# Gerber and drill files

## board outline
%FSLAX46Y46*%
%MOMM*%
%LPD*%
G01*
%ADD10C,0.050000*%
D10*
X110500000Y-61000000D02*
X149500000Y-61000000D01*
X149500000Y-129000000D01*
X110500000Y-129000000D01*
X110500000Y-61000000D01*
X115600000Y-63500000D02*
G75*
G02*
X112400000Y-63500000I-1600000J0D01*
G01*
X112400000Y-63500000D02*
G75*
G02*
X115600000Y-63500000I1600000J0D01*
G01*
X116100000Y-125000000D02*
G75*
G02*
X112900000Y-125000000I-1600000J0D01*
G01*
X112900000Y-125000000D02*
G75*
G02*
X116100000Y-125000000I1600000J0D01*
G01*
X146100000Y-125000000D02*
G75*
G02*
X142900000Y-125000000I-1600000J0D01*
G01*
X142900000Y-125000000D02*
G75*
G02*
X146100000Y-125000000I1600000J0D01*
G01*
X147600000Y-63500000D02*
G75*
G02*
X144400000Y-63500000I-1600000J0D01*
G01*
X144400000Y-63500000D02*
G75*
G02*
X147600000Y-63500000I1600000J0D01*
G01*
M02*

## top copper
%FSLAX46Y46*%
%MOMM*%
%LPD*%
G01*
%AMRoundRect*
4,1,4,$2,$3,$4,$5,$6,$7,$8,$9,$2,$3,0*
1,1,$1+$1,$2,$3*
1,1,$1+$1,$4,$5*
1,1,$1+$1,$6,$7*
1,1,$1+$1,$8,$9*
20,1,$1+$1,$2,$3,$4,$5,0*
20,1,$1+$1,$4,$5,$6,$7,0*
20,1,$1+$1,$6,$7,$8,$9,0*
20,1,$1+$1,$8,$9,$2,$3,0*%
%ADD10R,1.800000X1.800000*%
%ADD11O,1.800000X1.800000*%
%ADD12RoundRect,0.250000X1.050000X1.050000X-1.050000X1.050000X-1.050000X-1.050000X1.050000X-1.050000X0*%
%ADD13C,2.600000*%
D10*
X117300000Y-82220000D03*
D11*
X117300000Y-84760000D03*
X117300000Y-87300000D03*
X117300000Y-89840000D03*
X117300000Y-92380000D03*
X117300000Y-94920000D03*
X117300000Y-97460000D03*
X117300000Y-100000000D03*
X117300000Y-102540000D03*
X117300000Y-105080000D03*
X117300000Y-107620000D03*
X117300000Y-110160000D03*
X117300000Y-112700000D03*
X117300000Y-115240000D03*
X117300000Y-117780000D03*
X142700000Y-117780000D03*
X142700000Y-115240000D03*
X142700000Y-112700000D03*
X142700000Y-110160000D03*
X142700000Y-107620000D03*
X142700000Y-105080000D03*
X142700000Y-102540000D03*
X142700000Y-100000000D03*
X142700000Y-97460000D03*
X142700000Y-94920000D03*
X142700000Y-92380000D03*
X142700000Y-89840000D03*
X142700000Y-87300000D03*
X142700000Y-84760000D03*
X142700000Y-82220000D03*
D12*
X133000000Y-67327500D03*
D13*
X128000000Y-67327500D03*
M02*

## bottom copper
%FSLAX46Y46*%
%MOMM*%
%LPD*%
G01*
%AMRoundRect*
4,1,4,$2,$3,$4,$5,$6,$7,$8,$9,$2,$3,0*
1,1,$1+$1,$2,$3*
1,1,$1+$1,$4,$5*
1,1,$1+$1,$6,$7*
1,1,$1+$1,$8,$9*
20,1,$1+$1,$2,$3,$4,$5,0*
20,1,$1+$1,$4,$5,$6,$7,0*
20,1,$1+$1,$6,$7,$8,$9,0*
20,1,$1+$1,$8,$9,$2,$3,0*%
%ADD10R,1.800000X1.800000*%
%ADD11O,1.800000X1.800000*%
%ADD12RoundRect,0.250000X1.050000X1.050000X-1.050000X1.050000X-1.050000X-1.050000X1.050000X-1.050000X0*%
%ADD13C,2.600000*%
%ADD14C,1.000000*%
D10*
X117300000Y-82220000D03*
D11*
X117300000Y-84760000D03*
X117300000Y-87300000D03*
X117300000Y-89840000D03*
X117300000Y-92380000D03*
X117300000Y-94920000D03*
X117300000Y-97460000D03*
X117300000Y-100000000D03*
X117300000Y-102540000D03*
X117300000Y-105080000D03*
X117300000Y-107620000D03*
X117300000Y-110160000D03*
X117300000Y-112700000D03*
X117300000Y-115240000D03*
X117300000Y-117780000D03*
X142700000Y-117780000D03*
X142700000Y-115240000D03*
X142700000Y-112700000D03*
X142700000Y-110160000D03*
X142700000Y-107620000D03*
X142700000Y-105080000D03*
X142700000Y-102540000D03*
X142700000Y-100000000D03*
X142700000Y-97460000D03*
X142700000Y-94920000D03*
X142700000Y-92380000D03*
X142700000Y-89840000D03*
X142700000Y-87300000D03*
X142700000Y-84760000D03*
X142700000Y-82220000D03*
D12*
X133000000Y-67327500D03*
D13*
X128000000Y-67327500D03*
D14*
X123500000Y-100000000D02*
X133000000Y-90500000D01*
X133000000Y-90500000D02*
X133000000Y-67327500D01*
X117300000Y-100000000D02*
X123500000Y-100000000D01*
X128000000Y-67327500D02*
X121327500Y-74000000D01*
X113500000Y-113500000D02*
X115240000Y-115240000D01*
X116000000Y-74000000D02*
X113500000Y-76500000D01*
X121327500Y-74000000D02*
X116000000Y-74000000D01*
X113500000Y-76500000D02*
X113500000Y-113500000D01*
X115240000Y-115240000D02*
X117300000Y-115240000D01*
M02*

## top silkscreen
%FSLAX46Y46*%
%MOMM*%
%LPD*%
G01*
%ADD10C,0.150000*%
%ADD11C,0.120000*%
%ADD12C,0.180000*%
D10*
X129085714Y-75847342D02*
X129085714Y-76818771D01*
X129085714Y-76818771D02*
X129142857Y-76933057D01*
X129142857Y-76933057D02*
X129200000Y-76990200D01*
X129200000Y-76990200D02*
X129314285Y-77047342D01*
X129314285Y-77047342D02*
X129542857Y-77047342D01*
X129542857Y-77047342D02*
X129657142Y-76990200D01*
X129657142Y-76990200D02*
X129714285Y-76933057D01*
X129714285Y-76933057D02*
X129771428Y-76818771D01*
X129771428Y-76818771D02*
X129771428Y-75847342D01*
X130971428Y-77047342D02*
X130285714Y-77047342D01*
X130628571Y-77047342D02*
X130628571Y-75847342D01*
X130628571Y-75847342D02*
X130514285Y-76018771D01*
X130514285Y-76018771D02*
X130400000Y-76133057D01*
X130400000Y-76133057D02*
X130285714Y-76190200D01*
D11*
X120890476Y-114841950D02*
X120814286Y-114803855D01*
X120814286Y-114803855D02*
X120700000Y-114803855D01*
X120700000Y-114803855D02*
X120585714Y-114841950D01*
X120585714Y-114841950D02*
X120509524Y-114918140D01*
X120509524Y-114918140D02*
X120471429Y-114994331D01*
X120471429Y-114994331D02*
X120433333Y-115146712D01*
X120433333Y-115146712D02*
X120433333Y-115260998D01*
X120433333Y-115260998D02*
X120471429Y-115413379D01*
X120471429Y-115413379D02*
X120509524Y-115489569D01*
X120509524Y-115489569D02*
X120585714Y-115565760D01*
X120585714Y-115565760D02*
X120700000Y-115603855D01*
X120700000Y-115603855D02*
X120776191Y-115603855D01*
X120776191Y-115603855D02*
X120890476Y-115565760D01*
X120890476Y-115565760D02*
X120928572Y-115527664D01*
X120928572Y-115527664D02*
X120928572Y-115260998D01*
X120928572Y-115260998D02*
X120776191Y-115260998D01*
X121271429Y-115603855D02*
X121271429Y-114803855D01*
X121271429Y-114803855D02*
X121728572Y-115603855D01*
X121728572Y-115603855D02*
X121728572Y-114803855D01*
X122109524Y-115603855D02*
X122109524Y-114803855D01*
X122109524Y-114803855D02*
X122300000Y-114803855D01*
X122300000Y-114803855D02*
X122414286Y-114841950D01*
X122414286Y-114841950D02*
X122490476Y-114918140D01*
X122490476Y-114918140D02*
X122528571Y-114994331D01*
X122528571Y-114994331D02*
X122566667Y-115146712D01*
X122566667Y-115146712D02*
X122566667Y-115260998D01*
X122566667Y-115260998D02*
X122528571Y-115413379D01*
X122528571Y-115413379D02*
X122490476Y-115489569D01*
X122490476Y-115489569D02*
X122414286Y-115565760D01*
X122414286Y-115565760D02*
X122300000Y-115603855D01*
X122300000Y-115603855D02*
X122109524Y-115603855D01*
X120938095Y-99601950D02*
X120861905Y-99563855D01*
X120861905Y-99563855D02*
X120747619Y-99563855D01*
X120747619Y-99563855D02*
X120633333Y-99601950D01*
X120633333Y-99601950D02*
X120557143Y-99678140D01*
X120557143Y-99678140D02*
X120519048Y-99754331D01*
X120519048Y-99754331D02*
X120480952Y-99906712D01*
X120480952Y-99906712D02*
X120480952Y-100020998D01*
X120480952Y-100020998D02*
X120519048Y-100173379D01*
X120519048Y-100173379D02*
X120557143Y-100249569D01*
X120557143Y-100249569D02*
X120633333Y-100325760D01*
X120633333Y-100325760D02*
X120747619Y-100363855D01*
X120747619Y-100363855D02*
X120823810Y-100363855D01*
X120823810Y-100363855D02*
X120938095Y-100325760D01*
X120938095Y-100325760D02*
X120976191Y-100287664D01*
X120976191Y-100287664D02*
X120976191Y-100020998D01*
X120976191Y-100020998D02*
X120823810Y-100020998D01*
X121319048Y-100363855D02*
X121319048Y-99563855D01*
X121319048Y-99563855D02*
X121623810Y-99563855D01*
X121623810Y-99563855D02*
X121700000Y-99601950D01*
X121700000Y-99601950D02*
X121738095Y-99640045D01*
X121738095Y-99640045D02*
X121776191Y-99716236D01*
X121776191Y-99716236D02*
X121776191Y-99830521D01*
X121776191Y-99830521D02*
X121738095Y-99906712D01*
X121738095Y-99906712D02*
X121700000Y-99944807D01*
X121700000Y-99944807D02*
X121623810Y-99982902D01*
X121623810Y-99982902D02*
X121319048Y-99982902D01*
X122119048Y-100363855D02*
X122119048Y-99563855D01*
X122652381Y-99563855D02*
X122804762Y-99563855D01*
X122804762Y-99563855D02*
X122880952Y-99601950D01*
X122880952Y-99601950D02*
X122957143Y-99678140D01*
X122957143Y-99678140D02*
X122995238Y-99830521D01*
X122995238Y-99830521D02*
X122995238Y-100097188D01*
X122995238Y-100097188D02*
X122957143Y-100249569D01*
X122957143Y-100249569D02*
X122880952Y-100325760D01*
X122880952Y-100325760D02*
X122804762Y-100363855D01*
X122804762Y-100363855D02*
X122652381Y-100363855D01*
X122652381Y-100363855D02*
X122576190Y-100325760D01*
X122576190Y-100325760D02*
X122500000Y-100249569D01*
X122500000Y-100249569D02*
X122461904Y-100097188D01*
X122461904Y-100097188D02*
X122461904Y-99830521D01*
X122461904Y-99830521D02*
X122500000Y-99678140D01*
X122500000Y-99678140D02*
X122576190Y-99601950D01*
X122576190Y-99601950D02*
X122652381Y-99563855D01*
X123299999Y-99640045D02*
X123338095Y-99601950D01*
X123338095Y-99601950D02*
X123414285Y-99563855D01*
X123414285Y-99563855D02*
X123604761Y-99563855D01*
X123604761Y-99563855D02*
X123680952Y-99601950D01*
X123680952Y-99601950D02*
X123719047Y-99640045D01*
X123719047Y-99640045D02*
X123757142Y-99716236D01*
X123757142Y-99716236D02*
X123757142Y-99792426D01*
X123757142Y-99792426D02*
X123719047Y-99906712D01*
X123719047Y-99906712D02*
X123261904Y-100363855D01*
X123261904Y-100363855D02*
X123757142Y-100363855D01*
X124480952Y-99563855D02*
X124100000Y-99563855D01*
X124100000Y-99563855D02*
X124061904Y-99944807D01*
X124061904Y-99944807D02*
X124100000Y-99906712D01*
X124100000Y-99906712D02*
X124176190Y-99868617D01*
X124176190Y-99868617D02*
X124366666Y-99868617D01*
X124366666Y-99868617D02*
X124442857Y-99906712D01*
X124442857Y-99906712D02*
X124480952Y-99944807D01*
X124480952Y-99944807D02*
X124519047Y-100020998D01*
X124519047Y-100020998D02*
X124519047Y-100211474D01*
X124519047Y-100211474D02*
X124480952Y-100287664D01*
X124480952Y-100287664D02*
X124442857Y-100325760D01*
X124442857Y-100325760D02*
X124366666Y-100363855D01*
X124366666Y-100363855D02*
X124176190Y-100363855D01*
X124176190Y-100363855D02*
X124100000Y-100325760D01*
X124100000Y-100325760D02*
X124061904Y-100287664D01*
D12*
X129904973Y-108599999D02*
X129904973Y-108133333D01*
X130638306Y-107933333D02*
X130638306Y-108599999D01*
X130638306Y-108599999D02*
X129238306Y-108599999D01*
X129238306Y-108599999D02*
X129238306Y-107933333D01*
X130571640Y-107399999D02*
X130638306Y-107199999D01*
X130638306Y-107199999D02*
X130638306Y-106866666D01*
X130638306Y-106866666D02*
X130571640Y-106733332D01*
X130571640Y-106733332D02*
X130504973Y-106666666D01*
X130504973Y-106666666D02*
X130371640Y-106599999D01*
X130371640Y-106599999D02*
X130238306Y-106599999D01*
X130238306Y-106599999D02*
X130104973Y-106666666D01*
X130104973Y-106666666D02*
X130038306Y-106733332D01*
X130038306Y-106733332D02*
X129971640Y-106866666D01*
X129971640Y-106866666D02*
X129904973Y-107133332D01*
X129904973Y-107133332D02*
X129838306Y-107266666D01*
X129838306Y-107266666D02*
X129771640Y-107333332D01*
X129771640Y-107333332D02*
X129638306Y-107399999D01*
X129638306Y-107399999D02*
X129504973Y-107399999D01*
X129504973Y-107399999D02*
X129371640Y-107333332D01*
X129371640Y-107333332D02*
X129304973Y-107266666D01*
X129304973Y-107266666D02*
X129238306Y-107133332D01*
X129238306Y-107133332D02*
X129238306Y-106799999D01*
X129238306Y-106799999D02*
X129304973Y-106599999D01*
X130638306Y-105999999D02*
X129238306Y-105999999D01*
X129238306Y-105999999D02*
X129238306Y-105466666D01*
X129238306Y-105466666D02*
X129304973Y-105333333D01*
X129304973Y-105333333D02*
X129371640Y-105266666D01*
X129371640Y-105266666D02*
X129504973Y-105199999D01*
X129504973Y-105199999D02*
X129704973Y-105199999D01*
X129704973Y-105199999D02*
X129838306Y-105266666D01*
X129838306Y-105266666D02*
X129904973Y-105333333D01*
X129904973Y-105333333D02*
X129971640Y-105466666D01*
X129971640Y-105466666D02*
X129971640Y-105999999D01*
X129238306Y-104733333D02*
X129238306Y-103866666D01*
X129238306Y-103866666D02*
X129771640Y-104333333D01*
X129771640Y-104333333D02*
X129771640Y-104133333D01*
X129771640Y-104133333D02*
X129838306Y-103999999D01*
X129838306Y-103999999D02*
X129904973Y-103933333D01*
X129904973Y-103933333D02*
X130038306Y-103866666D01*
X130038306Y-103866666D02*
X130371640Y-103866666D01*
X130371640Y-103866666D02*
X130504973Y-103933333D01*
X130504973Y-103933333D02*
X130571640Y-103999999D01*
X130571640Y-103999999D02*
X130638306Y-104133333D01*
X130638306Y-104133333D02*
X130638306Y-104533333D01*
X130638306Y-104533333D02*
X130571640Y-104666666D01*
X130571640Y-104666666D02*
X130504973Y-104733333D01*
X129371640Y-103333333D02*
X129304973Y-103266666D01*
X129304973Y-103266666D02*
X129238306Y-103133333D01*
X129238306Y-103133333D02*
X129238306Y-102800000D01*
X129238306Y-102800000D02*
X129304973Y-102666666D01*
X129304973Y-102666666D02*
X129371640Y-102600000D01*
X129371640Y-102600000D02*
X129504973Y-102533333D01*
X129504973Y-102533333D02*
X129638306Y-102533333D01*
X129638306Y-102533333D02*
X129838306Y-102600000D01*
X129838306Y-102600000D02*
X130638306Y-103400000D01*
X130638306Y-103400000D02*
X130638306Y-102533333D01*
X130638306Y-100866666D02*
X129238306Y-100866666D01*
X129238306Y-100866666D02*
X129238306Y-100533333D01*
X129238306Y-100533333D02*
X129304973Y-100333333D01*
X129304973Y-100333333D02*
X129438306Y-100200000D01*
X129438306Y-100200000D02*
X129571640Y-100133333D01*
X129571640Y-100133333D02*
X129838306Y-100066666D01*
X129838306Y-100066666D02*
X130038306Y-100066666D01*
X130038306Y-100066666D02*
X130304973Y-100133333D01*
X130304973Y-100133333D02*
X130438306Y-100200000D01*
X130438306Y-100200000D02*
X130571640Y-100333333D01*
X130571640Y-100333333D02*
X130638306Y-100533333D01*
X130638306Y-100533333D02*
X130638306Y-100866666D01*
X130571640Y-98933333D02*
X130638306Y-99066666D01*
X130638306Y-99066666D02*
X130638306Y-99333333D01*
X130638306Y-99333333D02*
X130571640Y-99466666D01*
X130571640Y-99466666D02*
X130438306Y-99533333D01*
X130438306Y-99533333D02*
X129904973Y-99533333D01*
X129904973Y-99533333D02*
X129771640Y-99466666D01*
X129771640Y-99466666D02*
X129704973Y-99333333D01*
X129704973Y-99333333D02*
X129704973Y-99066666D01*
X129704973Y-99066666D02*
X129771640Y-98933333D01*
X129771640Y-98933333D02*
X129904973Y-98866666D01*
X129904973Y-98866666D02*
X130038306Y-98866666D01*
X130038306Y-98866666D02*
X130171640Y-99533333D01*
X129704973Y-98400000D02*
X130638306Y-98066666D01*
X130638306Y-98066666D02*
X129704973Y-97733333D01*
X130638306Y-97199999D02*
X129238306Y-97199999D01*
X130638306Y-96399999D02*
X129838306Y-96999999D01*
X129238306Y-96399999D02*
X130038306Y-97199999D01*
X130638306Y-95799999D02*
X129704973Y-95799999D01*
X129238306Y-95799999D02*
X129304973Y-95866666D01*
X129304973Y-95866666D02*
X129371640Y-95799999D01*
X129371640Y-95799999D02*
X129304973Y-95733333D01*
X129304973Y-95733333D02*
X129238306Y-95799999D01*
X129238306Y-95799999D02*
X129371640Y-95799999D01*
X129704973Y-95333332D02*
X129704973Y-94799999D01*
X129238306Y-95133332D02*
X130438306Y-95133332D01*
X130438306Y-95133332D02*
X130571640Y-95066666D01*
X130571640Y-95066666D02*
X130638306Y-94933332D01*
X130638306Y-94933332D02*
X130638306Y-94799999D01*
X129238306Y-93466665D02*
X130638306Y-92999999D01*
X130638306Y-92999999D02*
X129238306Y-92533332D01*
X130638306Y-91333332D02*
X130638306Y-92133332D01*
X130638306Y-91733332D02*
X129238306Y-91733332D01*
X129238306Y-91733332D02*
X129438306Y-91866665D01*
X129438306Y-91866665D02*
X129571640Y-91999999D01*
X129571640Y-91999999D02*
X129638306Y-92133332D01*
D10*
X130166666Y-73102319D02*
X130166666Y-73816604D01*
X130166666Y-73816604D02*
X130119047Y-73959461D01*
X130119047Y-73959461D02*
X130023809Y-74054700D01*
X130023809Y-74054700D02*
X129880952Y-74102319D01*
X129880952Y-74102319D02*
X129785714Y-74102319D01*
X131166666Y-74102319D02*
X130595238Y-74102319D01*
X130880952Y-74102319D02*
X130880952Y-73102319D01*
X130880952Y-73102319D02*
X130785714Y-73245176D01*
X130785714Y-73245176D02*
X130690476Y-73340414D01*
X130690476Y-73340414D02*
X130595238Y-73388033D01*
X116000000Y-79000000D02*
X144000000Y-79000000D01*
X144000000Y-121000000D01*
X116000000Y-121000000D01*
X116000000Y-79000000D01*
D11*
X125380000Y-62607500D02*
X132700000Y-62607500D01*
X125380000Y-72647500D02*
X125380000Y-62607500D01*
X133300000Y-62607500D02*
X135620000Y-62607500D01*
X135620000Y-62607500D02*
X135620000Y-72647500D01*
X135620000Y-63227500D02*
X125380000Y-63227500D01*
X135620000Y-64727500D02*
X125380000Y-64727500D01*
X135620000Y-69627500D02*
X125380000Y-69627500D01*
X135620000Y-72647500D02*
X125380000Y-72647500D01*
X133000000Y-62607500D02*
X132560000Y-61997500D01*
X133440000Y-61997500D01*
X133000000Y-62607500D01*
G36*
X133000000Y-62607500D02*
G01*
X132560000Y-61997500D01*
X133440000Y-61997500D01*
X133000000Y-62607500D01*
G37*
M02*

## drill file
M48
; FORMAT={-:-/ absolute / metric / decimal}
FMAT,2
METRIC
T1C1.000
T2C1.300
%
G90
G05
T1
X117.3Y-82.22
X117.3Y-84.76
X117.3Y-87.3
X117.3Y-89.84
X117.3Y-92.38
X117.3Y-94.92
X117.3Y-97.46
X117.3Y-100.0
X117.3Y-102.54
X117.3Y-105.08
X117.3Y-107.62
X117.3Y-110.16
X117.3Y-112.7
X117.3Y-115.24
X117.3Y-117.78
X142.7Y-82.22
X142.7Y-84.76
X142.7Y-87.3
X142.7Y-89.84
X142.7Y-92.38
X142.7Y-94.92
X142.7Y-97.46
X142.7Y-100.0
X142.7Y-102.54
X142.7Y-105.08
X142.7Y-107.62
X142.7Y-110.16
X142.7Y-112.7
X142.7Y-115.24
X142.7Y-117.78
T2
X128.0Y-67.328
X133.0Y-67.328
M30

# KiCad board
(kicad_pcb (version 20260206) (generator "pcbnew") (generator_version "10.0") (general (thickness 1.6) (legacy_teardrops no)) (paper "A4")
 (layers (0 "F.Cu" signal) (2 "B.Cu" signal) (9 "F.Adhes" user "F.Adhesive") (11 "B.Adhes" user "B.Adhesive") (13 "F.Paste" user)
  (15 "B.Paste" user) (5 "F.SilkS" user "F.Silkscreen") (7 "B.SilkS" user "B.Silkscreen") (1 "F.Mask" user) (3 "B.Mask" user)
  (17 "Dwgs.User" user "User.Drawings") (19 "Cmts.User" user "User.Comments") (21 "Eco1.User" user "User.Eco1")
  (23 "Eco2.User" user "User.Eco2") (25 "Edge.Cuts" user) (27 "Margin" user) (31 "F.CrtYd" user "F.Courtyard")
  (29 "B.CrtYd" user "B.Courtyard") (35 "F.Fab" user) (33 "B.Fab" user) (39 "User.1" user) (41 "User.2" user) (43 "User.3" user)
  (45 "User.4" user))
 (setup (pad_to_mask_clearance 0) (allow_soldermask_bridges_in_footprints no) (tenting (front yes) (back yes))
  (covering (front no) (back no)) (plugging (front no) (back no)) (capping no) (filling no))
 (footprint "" (layer "F.Cu") (at 130 100)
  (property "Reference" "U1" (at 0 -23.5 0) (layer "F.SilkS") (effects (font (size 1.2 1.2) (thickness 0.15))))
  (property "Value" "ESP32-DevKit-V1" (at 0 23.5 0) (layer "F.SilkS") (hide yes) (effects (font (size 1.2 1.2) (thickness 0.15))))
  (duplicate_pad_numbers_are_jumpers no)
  (fp_rect (start -14 -21) (end 14 21) (stroke (width 0.15) (type default)) (fill no) (layer "F.SilkS"))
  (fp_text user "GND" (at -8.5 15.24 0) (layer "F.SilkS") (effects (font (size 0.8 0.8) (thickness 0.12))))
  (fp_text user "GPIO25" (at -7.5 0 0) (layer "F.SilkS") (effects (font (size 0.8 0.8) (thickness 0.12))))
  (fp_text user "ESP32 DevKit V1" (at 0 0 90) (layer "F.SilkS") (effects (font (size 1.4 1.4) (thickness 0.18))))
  (pad "1" thru_hole rect (at -12.7 -17.78) (size 1.8 1.8) (drill 1) (layers "*.Cu" "*.Mask") (remove_unused_layers no)
   (thermal_bridge_angle 45))
  (pad "2" thru_hole oval (at -12.7 -15.24) (size 1.8 1.8) (drill 1) (layers "*.Cu" "*.Mask") (remove_unused_layers no)
   (thermal_bridge_angle 45))
  (pad "3" thru_hole oval (at -12.7 -12.7) (size 1.8 1.8) (drill 1) (layers "*.Cu" "*.Mask") (remove_unused_layers no)
   (thermal_bridge_angle 45))
  (pad "4" thru_hole oval (at -12.7 -10.16) (size 1.8 1.8) (drill 1) (layers "*.Cu" "*.Mask") (remove_unused_layers no)
   (thermal_bridge_angle 45))
  (pad "5" thru_hole oval (at -12.7 -7.62) (size 1.8 1.8) (drill 1) (layers "*.Cu" "*.Mask") (remove_unused_layers no)
   (thermal_bridge_angle 45))
  (pad "6" thru_hole oval (at -12.7 -5.08) (size 1.8 1.8) (drill 1) (layers "*.Cu" "*.Mask") (remove_unused_layers no)
   (thermal_bridge_angle 45))
  (pad "7" thru_hole oval (at -12.7 -2.54) (size 1.8 1.8) (drill 1) (layers "*.Cu" "*.Mask") (remove_unused_layers no)
   (thermal_bridge_angle 45))
  (pad "8" thru_hole oval (at -12.7 0) (size 1.8 1.8) (drill 1) (layers "*.Cu" "*.Mask") (remove_unused_layers no) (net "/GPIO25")
   (thermal_bridge_angle 45))
  (pad "9" thru_hole oval (at -12.7 2.54) (size 1.8 1.8) (drill 1) (layers "*.Cu" "*.Mask") (remove_unused_layers no)
   (thermal_bridge_angle 45))
  (pad "10" thru_hole oval (at -12.7 5.08) (size 1.8 1.8) (drill 1) (layers "*.Cu" "*.Mask") (remove_unused_layers no)
   (thermal_bridge_angle 45))
  (pad "11" thru_hole oval (at -12.7 7.62) (size 1.8 1.8) (drill 1) (layers "*.Cu" "*.Mask") (remove_unused_layers no)
   (thermal_bridge_angle 45))
  (pad "12" thru_hole oval (at -12.7 10.16) (size 1.8 1.8) (drill 1) (layers "*.Cu" "*.Mask") (remove_unused_layers no)
   (thermal_bridge_angle 45))
  (pad "13" thru_hole oval (at -12.7 12.7) (size 1.8 1.8) (drill 1) (layers "*.Cu" "*.Mask") (remove_unused_layers no)
   (thermal_bridge_angle 45))
  (pad "14" thru_hole oval (at -12.7 15.24) (size 1.8 1.8) (drill 1) (layers "*.Cu" "*.Mask") (remove_unused_layers no) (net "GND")
   (thermal_bridge_angle 45))
  (pad "15" thru_hole oval (at -12.7 17.78) (size 1.8 1.8) (drill 1) (layers "*.Cu" "*.Mask") (remove_unused_layers no)
   (thermal_bridge_angle 45))
  (pad "16" thru_hole oval (at 12.7 17.78) (size 1.8 1.8) (drill 1) (layers "*.Cu" "*.Mask") (remove_unused_layers no)
   (thermal_bridge_angle 45))
  (pad "17" thru_hole oval (at 12.7 15.24) (size 1.8 1.8) (drill 1) (layers "*.Cu" "*.Mask") (remove_unused_layers no)
   (thermal_bridge_angle 45))
  (pad "18" thru_hole oval (at 12.7 12.7) (size 1.8 1.8) (drill 1) (layers "*.Cu" "*.Mask") (remove_unused_layers no)
   (thermal_bridge_angle 45))
  (pad "19" thru_hole oval (at 12.7 10.16) (size 1.8 1.8) (drill 1) (layers "*.Cu" "*.Mask") (remove_unused_layers no)
   (thermal_bridge_angle 45))
  (pad "20" thru_hole oval (at 12.7 7.62) (size 1.8 1.8) (drill 1) (layers "*.Cu" "*.Mask") (remove_unused_layers no)
   (thermal_bridge_angle 45))
  (pad "21" thru_hole oval (at 12.7 5.08) (size 1.8 1.8) (drill 1) (layers "*.Cu" "*.Mask") (remove_unused_layers no)
   (thermal_bridge_angle 45))
  (pad "22" thru_hole oval (at 12.7 2.54) (size 1.8 1.8) (drill 1) (layers "*.Cu" "*.Mask") (remove_unused_layers no)
   (thermal_bridge_angle 45))
  (pad "23" thru_hole oval (at 12.7 0) (size 1.8 1.8) (drill 1) (layers "*.Cu" "*.Mask") (remove_unused_layers no) (thermal_bridge_angle 45))
  (pad "24" thru_hole oval (at 12.7 -2.54) (size 1.8 1.8) (drill 1) (layers "*.Cu" "*.Mask") (remove_unused_layers no)
   (thermal_bridge_angle 45))
  (pad "25" thru_hole oval (at 12.7 -5.08) (size 1.8 1.8) (drill 1) (layers "*.Cu" "*.Mask") (remove_unused_layers no)
   (thermal_bridge_angle 45))
  (pad "26" thru_hole oval (at 12.7 -7.62) (size 1.8 1.8) (drill 1) (layers "*.Cu" "*.Mask") (remove_unused_layers no)
   (thermal_bridge_angle 45))
  (pad "27" thru_hole oval (at 12.7 -10.16) (size 1.8 1.8) (drill 1) (layers "*.Cu" "*.Mask") (remove_unused_layers no)
   (thermal_bridge_angle 45))
  (pad "28" thru_hole oval (at 12.7 -12.7) (size 1.8 1.8) (drill 1) (layers "*.Cu" "*.Mask") (remove_unused_layers no)
   (thermal_bridge_angle 45))
  (pad "29" thru_hole oval (at 12.7 -15.24) (size 1.8 1.8) (drill 1) (layers "*.Cu" "*.Mask") (remove_unused_layers no)
   (thermal_bridge_angle 45))
  (pad "30" thru_hole oval (at 12.7 -17.78) (size 1.8 1.8) (drill 1) (layers "*.Cu" "*.Mask") (remove_unused_layers no)
   (thermal_bridge_angle 45)))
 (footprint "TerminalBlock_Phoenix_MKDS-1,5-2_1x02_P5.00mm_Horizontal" (layer "F.Cu") (at 133 67.3275 180)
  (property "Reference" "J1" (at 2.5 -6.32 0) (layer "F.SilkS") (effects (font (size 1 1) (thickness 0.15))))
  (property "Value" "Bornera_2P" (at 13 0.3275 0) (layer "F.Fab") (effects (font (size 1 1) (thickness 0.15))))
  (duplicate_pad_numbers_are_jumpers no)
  (fp_line (start 7.62 4.72) (end 0.3 4.72) (stroke (width 0.12) (type solid)) (layer "F.SilkS"))
  (fp_line (start 7.62 -5.32) (end 7.62 4.72) (stroke (width 0.12) (type solid)) (layer "F.SilkS"))
  (fp_line (start -0.3 4.72) (end -2.62 4.72) (stroke (width 0.12) (type solid)) (layer "F.SilkS"))
  (fp_line (start -2.62 4.72) (end -2.62 -5.32) (stroke (width 0.12) (type solid)) (layer "F.SilkS"))
  (fp_line (start -2.62 4.1) (end 7.62 4.1) (stroke (width 0.12) (type solid)) (layer "F.SilkS"))
  (fp_line (start -2.62 2.6) (end 7.62 2.6) (stroke (width 0.12) (type solid)) (layer "F.SilkS"))
  (fp_line (start -2.62 -2.3) (end 7.62 -2.3) (stroke (width 0.12) (type solid)) (layer "F.SilkS"))
  (fp_line (start -2.62 -5.32) (end 7.62 -5.32) (stroke (width 0.12) (type solid)) (layer "F.SilkS"))
  (fp_poly (pts (xy 0 4.72) (xy 0.44 5.33) (xy -0.44 5.33)) (stroke (width 0.12) (type solid)) (fill yes) (layer "F.SilkS"))
  (pad "1" thru_hole roundrect (at 0 0 180) (size 2.6 2.6) (drill 1.3) (layers "*.Cu" "*.Mask") (remove_unused_layers no)
   (roundrect_rratio 0.096154) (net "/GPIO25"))
  (pad "2" thru_hole circle (at 5 0 180) (size 2.6 2.6) (drill 1.3) (layers "*.Cu" "*.Mask") (remove_unused_layers no) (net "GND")))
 (gr_rect (start 110.5 61) (end 149.5 129) (stroke (width 0.05) (type default)) (fill no) (layer "Edge.Cuts"))
 (gr_circle (center 114 63.5) (end 115.6 63.5) (stroke (width 0.05) (type solid)) (fill no) (layer "Edge.Cuts"))
 (gr_circle (center 114.5 125) (end 116.1 125) (stroke (width 0.05) (type solid)) (fill no) (layer "Edge.Cuts"))
 (gr_circle (center 144.5 125) (end 146.1 125) (stroke (width 0.05) (type solid)) (fill no) (layer "Edge.Cuts"))
 (gr_circle (center 146 63.5) (end 147.6 63.5) (stroke (width 0.05) (type solid)) (fill no) (layer "Edge.Cuts"))
 (segment (start 123.5 100) (end 133 90.5) (width 1) (layer "B.Cu") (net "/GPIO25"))
 (segment (start 133 90.5) (end 133 67.3275) (width 1) (layer "B.Cu") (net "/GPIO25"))
 (segment (start 117.3 100) (end 123.5 100) (width 1) (layer "B.Cu") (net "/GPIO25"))
 (segment (start 128 67.3275) (end 121.3275 74) (width 1) (layer "B.Cu") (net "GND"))
 (segment (start 113.5 113.5) (end 115.24 115.24) (width 1) (layer "B.Cu") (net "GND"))
 (segment (start 116 74) (end 113.5 76.5) (width 1) (layer "B.Cu") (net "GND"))
 (segment (start 121.3275 74) (end 116 74) (width 1) (layer "B.Cu") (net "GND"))
 (segment (start 113.5 76.5) (end 113.5 113.5) (width 1) (layer "B.Cu") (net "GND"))
 (segment (start 115.24 115.24) (end 117.3 115.24) (width 1) (layer "B.Cu") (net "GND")))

